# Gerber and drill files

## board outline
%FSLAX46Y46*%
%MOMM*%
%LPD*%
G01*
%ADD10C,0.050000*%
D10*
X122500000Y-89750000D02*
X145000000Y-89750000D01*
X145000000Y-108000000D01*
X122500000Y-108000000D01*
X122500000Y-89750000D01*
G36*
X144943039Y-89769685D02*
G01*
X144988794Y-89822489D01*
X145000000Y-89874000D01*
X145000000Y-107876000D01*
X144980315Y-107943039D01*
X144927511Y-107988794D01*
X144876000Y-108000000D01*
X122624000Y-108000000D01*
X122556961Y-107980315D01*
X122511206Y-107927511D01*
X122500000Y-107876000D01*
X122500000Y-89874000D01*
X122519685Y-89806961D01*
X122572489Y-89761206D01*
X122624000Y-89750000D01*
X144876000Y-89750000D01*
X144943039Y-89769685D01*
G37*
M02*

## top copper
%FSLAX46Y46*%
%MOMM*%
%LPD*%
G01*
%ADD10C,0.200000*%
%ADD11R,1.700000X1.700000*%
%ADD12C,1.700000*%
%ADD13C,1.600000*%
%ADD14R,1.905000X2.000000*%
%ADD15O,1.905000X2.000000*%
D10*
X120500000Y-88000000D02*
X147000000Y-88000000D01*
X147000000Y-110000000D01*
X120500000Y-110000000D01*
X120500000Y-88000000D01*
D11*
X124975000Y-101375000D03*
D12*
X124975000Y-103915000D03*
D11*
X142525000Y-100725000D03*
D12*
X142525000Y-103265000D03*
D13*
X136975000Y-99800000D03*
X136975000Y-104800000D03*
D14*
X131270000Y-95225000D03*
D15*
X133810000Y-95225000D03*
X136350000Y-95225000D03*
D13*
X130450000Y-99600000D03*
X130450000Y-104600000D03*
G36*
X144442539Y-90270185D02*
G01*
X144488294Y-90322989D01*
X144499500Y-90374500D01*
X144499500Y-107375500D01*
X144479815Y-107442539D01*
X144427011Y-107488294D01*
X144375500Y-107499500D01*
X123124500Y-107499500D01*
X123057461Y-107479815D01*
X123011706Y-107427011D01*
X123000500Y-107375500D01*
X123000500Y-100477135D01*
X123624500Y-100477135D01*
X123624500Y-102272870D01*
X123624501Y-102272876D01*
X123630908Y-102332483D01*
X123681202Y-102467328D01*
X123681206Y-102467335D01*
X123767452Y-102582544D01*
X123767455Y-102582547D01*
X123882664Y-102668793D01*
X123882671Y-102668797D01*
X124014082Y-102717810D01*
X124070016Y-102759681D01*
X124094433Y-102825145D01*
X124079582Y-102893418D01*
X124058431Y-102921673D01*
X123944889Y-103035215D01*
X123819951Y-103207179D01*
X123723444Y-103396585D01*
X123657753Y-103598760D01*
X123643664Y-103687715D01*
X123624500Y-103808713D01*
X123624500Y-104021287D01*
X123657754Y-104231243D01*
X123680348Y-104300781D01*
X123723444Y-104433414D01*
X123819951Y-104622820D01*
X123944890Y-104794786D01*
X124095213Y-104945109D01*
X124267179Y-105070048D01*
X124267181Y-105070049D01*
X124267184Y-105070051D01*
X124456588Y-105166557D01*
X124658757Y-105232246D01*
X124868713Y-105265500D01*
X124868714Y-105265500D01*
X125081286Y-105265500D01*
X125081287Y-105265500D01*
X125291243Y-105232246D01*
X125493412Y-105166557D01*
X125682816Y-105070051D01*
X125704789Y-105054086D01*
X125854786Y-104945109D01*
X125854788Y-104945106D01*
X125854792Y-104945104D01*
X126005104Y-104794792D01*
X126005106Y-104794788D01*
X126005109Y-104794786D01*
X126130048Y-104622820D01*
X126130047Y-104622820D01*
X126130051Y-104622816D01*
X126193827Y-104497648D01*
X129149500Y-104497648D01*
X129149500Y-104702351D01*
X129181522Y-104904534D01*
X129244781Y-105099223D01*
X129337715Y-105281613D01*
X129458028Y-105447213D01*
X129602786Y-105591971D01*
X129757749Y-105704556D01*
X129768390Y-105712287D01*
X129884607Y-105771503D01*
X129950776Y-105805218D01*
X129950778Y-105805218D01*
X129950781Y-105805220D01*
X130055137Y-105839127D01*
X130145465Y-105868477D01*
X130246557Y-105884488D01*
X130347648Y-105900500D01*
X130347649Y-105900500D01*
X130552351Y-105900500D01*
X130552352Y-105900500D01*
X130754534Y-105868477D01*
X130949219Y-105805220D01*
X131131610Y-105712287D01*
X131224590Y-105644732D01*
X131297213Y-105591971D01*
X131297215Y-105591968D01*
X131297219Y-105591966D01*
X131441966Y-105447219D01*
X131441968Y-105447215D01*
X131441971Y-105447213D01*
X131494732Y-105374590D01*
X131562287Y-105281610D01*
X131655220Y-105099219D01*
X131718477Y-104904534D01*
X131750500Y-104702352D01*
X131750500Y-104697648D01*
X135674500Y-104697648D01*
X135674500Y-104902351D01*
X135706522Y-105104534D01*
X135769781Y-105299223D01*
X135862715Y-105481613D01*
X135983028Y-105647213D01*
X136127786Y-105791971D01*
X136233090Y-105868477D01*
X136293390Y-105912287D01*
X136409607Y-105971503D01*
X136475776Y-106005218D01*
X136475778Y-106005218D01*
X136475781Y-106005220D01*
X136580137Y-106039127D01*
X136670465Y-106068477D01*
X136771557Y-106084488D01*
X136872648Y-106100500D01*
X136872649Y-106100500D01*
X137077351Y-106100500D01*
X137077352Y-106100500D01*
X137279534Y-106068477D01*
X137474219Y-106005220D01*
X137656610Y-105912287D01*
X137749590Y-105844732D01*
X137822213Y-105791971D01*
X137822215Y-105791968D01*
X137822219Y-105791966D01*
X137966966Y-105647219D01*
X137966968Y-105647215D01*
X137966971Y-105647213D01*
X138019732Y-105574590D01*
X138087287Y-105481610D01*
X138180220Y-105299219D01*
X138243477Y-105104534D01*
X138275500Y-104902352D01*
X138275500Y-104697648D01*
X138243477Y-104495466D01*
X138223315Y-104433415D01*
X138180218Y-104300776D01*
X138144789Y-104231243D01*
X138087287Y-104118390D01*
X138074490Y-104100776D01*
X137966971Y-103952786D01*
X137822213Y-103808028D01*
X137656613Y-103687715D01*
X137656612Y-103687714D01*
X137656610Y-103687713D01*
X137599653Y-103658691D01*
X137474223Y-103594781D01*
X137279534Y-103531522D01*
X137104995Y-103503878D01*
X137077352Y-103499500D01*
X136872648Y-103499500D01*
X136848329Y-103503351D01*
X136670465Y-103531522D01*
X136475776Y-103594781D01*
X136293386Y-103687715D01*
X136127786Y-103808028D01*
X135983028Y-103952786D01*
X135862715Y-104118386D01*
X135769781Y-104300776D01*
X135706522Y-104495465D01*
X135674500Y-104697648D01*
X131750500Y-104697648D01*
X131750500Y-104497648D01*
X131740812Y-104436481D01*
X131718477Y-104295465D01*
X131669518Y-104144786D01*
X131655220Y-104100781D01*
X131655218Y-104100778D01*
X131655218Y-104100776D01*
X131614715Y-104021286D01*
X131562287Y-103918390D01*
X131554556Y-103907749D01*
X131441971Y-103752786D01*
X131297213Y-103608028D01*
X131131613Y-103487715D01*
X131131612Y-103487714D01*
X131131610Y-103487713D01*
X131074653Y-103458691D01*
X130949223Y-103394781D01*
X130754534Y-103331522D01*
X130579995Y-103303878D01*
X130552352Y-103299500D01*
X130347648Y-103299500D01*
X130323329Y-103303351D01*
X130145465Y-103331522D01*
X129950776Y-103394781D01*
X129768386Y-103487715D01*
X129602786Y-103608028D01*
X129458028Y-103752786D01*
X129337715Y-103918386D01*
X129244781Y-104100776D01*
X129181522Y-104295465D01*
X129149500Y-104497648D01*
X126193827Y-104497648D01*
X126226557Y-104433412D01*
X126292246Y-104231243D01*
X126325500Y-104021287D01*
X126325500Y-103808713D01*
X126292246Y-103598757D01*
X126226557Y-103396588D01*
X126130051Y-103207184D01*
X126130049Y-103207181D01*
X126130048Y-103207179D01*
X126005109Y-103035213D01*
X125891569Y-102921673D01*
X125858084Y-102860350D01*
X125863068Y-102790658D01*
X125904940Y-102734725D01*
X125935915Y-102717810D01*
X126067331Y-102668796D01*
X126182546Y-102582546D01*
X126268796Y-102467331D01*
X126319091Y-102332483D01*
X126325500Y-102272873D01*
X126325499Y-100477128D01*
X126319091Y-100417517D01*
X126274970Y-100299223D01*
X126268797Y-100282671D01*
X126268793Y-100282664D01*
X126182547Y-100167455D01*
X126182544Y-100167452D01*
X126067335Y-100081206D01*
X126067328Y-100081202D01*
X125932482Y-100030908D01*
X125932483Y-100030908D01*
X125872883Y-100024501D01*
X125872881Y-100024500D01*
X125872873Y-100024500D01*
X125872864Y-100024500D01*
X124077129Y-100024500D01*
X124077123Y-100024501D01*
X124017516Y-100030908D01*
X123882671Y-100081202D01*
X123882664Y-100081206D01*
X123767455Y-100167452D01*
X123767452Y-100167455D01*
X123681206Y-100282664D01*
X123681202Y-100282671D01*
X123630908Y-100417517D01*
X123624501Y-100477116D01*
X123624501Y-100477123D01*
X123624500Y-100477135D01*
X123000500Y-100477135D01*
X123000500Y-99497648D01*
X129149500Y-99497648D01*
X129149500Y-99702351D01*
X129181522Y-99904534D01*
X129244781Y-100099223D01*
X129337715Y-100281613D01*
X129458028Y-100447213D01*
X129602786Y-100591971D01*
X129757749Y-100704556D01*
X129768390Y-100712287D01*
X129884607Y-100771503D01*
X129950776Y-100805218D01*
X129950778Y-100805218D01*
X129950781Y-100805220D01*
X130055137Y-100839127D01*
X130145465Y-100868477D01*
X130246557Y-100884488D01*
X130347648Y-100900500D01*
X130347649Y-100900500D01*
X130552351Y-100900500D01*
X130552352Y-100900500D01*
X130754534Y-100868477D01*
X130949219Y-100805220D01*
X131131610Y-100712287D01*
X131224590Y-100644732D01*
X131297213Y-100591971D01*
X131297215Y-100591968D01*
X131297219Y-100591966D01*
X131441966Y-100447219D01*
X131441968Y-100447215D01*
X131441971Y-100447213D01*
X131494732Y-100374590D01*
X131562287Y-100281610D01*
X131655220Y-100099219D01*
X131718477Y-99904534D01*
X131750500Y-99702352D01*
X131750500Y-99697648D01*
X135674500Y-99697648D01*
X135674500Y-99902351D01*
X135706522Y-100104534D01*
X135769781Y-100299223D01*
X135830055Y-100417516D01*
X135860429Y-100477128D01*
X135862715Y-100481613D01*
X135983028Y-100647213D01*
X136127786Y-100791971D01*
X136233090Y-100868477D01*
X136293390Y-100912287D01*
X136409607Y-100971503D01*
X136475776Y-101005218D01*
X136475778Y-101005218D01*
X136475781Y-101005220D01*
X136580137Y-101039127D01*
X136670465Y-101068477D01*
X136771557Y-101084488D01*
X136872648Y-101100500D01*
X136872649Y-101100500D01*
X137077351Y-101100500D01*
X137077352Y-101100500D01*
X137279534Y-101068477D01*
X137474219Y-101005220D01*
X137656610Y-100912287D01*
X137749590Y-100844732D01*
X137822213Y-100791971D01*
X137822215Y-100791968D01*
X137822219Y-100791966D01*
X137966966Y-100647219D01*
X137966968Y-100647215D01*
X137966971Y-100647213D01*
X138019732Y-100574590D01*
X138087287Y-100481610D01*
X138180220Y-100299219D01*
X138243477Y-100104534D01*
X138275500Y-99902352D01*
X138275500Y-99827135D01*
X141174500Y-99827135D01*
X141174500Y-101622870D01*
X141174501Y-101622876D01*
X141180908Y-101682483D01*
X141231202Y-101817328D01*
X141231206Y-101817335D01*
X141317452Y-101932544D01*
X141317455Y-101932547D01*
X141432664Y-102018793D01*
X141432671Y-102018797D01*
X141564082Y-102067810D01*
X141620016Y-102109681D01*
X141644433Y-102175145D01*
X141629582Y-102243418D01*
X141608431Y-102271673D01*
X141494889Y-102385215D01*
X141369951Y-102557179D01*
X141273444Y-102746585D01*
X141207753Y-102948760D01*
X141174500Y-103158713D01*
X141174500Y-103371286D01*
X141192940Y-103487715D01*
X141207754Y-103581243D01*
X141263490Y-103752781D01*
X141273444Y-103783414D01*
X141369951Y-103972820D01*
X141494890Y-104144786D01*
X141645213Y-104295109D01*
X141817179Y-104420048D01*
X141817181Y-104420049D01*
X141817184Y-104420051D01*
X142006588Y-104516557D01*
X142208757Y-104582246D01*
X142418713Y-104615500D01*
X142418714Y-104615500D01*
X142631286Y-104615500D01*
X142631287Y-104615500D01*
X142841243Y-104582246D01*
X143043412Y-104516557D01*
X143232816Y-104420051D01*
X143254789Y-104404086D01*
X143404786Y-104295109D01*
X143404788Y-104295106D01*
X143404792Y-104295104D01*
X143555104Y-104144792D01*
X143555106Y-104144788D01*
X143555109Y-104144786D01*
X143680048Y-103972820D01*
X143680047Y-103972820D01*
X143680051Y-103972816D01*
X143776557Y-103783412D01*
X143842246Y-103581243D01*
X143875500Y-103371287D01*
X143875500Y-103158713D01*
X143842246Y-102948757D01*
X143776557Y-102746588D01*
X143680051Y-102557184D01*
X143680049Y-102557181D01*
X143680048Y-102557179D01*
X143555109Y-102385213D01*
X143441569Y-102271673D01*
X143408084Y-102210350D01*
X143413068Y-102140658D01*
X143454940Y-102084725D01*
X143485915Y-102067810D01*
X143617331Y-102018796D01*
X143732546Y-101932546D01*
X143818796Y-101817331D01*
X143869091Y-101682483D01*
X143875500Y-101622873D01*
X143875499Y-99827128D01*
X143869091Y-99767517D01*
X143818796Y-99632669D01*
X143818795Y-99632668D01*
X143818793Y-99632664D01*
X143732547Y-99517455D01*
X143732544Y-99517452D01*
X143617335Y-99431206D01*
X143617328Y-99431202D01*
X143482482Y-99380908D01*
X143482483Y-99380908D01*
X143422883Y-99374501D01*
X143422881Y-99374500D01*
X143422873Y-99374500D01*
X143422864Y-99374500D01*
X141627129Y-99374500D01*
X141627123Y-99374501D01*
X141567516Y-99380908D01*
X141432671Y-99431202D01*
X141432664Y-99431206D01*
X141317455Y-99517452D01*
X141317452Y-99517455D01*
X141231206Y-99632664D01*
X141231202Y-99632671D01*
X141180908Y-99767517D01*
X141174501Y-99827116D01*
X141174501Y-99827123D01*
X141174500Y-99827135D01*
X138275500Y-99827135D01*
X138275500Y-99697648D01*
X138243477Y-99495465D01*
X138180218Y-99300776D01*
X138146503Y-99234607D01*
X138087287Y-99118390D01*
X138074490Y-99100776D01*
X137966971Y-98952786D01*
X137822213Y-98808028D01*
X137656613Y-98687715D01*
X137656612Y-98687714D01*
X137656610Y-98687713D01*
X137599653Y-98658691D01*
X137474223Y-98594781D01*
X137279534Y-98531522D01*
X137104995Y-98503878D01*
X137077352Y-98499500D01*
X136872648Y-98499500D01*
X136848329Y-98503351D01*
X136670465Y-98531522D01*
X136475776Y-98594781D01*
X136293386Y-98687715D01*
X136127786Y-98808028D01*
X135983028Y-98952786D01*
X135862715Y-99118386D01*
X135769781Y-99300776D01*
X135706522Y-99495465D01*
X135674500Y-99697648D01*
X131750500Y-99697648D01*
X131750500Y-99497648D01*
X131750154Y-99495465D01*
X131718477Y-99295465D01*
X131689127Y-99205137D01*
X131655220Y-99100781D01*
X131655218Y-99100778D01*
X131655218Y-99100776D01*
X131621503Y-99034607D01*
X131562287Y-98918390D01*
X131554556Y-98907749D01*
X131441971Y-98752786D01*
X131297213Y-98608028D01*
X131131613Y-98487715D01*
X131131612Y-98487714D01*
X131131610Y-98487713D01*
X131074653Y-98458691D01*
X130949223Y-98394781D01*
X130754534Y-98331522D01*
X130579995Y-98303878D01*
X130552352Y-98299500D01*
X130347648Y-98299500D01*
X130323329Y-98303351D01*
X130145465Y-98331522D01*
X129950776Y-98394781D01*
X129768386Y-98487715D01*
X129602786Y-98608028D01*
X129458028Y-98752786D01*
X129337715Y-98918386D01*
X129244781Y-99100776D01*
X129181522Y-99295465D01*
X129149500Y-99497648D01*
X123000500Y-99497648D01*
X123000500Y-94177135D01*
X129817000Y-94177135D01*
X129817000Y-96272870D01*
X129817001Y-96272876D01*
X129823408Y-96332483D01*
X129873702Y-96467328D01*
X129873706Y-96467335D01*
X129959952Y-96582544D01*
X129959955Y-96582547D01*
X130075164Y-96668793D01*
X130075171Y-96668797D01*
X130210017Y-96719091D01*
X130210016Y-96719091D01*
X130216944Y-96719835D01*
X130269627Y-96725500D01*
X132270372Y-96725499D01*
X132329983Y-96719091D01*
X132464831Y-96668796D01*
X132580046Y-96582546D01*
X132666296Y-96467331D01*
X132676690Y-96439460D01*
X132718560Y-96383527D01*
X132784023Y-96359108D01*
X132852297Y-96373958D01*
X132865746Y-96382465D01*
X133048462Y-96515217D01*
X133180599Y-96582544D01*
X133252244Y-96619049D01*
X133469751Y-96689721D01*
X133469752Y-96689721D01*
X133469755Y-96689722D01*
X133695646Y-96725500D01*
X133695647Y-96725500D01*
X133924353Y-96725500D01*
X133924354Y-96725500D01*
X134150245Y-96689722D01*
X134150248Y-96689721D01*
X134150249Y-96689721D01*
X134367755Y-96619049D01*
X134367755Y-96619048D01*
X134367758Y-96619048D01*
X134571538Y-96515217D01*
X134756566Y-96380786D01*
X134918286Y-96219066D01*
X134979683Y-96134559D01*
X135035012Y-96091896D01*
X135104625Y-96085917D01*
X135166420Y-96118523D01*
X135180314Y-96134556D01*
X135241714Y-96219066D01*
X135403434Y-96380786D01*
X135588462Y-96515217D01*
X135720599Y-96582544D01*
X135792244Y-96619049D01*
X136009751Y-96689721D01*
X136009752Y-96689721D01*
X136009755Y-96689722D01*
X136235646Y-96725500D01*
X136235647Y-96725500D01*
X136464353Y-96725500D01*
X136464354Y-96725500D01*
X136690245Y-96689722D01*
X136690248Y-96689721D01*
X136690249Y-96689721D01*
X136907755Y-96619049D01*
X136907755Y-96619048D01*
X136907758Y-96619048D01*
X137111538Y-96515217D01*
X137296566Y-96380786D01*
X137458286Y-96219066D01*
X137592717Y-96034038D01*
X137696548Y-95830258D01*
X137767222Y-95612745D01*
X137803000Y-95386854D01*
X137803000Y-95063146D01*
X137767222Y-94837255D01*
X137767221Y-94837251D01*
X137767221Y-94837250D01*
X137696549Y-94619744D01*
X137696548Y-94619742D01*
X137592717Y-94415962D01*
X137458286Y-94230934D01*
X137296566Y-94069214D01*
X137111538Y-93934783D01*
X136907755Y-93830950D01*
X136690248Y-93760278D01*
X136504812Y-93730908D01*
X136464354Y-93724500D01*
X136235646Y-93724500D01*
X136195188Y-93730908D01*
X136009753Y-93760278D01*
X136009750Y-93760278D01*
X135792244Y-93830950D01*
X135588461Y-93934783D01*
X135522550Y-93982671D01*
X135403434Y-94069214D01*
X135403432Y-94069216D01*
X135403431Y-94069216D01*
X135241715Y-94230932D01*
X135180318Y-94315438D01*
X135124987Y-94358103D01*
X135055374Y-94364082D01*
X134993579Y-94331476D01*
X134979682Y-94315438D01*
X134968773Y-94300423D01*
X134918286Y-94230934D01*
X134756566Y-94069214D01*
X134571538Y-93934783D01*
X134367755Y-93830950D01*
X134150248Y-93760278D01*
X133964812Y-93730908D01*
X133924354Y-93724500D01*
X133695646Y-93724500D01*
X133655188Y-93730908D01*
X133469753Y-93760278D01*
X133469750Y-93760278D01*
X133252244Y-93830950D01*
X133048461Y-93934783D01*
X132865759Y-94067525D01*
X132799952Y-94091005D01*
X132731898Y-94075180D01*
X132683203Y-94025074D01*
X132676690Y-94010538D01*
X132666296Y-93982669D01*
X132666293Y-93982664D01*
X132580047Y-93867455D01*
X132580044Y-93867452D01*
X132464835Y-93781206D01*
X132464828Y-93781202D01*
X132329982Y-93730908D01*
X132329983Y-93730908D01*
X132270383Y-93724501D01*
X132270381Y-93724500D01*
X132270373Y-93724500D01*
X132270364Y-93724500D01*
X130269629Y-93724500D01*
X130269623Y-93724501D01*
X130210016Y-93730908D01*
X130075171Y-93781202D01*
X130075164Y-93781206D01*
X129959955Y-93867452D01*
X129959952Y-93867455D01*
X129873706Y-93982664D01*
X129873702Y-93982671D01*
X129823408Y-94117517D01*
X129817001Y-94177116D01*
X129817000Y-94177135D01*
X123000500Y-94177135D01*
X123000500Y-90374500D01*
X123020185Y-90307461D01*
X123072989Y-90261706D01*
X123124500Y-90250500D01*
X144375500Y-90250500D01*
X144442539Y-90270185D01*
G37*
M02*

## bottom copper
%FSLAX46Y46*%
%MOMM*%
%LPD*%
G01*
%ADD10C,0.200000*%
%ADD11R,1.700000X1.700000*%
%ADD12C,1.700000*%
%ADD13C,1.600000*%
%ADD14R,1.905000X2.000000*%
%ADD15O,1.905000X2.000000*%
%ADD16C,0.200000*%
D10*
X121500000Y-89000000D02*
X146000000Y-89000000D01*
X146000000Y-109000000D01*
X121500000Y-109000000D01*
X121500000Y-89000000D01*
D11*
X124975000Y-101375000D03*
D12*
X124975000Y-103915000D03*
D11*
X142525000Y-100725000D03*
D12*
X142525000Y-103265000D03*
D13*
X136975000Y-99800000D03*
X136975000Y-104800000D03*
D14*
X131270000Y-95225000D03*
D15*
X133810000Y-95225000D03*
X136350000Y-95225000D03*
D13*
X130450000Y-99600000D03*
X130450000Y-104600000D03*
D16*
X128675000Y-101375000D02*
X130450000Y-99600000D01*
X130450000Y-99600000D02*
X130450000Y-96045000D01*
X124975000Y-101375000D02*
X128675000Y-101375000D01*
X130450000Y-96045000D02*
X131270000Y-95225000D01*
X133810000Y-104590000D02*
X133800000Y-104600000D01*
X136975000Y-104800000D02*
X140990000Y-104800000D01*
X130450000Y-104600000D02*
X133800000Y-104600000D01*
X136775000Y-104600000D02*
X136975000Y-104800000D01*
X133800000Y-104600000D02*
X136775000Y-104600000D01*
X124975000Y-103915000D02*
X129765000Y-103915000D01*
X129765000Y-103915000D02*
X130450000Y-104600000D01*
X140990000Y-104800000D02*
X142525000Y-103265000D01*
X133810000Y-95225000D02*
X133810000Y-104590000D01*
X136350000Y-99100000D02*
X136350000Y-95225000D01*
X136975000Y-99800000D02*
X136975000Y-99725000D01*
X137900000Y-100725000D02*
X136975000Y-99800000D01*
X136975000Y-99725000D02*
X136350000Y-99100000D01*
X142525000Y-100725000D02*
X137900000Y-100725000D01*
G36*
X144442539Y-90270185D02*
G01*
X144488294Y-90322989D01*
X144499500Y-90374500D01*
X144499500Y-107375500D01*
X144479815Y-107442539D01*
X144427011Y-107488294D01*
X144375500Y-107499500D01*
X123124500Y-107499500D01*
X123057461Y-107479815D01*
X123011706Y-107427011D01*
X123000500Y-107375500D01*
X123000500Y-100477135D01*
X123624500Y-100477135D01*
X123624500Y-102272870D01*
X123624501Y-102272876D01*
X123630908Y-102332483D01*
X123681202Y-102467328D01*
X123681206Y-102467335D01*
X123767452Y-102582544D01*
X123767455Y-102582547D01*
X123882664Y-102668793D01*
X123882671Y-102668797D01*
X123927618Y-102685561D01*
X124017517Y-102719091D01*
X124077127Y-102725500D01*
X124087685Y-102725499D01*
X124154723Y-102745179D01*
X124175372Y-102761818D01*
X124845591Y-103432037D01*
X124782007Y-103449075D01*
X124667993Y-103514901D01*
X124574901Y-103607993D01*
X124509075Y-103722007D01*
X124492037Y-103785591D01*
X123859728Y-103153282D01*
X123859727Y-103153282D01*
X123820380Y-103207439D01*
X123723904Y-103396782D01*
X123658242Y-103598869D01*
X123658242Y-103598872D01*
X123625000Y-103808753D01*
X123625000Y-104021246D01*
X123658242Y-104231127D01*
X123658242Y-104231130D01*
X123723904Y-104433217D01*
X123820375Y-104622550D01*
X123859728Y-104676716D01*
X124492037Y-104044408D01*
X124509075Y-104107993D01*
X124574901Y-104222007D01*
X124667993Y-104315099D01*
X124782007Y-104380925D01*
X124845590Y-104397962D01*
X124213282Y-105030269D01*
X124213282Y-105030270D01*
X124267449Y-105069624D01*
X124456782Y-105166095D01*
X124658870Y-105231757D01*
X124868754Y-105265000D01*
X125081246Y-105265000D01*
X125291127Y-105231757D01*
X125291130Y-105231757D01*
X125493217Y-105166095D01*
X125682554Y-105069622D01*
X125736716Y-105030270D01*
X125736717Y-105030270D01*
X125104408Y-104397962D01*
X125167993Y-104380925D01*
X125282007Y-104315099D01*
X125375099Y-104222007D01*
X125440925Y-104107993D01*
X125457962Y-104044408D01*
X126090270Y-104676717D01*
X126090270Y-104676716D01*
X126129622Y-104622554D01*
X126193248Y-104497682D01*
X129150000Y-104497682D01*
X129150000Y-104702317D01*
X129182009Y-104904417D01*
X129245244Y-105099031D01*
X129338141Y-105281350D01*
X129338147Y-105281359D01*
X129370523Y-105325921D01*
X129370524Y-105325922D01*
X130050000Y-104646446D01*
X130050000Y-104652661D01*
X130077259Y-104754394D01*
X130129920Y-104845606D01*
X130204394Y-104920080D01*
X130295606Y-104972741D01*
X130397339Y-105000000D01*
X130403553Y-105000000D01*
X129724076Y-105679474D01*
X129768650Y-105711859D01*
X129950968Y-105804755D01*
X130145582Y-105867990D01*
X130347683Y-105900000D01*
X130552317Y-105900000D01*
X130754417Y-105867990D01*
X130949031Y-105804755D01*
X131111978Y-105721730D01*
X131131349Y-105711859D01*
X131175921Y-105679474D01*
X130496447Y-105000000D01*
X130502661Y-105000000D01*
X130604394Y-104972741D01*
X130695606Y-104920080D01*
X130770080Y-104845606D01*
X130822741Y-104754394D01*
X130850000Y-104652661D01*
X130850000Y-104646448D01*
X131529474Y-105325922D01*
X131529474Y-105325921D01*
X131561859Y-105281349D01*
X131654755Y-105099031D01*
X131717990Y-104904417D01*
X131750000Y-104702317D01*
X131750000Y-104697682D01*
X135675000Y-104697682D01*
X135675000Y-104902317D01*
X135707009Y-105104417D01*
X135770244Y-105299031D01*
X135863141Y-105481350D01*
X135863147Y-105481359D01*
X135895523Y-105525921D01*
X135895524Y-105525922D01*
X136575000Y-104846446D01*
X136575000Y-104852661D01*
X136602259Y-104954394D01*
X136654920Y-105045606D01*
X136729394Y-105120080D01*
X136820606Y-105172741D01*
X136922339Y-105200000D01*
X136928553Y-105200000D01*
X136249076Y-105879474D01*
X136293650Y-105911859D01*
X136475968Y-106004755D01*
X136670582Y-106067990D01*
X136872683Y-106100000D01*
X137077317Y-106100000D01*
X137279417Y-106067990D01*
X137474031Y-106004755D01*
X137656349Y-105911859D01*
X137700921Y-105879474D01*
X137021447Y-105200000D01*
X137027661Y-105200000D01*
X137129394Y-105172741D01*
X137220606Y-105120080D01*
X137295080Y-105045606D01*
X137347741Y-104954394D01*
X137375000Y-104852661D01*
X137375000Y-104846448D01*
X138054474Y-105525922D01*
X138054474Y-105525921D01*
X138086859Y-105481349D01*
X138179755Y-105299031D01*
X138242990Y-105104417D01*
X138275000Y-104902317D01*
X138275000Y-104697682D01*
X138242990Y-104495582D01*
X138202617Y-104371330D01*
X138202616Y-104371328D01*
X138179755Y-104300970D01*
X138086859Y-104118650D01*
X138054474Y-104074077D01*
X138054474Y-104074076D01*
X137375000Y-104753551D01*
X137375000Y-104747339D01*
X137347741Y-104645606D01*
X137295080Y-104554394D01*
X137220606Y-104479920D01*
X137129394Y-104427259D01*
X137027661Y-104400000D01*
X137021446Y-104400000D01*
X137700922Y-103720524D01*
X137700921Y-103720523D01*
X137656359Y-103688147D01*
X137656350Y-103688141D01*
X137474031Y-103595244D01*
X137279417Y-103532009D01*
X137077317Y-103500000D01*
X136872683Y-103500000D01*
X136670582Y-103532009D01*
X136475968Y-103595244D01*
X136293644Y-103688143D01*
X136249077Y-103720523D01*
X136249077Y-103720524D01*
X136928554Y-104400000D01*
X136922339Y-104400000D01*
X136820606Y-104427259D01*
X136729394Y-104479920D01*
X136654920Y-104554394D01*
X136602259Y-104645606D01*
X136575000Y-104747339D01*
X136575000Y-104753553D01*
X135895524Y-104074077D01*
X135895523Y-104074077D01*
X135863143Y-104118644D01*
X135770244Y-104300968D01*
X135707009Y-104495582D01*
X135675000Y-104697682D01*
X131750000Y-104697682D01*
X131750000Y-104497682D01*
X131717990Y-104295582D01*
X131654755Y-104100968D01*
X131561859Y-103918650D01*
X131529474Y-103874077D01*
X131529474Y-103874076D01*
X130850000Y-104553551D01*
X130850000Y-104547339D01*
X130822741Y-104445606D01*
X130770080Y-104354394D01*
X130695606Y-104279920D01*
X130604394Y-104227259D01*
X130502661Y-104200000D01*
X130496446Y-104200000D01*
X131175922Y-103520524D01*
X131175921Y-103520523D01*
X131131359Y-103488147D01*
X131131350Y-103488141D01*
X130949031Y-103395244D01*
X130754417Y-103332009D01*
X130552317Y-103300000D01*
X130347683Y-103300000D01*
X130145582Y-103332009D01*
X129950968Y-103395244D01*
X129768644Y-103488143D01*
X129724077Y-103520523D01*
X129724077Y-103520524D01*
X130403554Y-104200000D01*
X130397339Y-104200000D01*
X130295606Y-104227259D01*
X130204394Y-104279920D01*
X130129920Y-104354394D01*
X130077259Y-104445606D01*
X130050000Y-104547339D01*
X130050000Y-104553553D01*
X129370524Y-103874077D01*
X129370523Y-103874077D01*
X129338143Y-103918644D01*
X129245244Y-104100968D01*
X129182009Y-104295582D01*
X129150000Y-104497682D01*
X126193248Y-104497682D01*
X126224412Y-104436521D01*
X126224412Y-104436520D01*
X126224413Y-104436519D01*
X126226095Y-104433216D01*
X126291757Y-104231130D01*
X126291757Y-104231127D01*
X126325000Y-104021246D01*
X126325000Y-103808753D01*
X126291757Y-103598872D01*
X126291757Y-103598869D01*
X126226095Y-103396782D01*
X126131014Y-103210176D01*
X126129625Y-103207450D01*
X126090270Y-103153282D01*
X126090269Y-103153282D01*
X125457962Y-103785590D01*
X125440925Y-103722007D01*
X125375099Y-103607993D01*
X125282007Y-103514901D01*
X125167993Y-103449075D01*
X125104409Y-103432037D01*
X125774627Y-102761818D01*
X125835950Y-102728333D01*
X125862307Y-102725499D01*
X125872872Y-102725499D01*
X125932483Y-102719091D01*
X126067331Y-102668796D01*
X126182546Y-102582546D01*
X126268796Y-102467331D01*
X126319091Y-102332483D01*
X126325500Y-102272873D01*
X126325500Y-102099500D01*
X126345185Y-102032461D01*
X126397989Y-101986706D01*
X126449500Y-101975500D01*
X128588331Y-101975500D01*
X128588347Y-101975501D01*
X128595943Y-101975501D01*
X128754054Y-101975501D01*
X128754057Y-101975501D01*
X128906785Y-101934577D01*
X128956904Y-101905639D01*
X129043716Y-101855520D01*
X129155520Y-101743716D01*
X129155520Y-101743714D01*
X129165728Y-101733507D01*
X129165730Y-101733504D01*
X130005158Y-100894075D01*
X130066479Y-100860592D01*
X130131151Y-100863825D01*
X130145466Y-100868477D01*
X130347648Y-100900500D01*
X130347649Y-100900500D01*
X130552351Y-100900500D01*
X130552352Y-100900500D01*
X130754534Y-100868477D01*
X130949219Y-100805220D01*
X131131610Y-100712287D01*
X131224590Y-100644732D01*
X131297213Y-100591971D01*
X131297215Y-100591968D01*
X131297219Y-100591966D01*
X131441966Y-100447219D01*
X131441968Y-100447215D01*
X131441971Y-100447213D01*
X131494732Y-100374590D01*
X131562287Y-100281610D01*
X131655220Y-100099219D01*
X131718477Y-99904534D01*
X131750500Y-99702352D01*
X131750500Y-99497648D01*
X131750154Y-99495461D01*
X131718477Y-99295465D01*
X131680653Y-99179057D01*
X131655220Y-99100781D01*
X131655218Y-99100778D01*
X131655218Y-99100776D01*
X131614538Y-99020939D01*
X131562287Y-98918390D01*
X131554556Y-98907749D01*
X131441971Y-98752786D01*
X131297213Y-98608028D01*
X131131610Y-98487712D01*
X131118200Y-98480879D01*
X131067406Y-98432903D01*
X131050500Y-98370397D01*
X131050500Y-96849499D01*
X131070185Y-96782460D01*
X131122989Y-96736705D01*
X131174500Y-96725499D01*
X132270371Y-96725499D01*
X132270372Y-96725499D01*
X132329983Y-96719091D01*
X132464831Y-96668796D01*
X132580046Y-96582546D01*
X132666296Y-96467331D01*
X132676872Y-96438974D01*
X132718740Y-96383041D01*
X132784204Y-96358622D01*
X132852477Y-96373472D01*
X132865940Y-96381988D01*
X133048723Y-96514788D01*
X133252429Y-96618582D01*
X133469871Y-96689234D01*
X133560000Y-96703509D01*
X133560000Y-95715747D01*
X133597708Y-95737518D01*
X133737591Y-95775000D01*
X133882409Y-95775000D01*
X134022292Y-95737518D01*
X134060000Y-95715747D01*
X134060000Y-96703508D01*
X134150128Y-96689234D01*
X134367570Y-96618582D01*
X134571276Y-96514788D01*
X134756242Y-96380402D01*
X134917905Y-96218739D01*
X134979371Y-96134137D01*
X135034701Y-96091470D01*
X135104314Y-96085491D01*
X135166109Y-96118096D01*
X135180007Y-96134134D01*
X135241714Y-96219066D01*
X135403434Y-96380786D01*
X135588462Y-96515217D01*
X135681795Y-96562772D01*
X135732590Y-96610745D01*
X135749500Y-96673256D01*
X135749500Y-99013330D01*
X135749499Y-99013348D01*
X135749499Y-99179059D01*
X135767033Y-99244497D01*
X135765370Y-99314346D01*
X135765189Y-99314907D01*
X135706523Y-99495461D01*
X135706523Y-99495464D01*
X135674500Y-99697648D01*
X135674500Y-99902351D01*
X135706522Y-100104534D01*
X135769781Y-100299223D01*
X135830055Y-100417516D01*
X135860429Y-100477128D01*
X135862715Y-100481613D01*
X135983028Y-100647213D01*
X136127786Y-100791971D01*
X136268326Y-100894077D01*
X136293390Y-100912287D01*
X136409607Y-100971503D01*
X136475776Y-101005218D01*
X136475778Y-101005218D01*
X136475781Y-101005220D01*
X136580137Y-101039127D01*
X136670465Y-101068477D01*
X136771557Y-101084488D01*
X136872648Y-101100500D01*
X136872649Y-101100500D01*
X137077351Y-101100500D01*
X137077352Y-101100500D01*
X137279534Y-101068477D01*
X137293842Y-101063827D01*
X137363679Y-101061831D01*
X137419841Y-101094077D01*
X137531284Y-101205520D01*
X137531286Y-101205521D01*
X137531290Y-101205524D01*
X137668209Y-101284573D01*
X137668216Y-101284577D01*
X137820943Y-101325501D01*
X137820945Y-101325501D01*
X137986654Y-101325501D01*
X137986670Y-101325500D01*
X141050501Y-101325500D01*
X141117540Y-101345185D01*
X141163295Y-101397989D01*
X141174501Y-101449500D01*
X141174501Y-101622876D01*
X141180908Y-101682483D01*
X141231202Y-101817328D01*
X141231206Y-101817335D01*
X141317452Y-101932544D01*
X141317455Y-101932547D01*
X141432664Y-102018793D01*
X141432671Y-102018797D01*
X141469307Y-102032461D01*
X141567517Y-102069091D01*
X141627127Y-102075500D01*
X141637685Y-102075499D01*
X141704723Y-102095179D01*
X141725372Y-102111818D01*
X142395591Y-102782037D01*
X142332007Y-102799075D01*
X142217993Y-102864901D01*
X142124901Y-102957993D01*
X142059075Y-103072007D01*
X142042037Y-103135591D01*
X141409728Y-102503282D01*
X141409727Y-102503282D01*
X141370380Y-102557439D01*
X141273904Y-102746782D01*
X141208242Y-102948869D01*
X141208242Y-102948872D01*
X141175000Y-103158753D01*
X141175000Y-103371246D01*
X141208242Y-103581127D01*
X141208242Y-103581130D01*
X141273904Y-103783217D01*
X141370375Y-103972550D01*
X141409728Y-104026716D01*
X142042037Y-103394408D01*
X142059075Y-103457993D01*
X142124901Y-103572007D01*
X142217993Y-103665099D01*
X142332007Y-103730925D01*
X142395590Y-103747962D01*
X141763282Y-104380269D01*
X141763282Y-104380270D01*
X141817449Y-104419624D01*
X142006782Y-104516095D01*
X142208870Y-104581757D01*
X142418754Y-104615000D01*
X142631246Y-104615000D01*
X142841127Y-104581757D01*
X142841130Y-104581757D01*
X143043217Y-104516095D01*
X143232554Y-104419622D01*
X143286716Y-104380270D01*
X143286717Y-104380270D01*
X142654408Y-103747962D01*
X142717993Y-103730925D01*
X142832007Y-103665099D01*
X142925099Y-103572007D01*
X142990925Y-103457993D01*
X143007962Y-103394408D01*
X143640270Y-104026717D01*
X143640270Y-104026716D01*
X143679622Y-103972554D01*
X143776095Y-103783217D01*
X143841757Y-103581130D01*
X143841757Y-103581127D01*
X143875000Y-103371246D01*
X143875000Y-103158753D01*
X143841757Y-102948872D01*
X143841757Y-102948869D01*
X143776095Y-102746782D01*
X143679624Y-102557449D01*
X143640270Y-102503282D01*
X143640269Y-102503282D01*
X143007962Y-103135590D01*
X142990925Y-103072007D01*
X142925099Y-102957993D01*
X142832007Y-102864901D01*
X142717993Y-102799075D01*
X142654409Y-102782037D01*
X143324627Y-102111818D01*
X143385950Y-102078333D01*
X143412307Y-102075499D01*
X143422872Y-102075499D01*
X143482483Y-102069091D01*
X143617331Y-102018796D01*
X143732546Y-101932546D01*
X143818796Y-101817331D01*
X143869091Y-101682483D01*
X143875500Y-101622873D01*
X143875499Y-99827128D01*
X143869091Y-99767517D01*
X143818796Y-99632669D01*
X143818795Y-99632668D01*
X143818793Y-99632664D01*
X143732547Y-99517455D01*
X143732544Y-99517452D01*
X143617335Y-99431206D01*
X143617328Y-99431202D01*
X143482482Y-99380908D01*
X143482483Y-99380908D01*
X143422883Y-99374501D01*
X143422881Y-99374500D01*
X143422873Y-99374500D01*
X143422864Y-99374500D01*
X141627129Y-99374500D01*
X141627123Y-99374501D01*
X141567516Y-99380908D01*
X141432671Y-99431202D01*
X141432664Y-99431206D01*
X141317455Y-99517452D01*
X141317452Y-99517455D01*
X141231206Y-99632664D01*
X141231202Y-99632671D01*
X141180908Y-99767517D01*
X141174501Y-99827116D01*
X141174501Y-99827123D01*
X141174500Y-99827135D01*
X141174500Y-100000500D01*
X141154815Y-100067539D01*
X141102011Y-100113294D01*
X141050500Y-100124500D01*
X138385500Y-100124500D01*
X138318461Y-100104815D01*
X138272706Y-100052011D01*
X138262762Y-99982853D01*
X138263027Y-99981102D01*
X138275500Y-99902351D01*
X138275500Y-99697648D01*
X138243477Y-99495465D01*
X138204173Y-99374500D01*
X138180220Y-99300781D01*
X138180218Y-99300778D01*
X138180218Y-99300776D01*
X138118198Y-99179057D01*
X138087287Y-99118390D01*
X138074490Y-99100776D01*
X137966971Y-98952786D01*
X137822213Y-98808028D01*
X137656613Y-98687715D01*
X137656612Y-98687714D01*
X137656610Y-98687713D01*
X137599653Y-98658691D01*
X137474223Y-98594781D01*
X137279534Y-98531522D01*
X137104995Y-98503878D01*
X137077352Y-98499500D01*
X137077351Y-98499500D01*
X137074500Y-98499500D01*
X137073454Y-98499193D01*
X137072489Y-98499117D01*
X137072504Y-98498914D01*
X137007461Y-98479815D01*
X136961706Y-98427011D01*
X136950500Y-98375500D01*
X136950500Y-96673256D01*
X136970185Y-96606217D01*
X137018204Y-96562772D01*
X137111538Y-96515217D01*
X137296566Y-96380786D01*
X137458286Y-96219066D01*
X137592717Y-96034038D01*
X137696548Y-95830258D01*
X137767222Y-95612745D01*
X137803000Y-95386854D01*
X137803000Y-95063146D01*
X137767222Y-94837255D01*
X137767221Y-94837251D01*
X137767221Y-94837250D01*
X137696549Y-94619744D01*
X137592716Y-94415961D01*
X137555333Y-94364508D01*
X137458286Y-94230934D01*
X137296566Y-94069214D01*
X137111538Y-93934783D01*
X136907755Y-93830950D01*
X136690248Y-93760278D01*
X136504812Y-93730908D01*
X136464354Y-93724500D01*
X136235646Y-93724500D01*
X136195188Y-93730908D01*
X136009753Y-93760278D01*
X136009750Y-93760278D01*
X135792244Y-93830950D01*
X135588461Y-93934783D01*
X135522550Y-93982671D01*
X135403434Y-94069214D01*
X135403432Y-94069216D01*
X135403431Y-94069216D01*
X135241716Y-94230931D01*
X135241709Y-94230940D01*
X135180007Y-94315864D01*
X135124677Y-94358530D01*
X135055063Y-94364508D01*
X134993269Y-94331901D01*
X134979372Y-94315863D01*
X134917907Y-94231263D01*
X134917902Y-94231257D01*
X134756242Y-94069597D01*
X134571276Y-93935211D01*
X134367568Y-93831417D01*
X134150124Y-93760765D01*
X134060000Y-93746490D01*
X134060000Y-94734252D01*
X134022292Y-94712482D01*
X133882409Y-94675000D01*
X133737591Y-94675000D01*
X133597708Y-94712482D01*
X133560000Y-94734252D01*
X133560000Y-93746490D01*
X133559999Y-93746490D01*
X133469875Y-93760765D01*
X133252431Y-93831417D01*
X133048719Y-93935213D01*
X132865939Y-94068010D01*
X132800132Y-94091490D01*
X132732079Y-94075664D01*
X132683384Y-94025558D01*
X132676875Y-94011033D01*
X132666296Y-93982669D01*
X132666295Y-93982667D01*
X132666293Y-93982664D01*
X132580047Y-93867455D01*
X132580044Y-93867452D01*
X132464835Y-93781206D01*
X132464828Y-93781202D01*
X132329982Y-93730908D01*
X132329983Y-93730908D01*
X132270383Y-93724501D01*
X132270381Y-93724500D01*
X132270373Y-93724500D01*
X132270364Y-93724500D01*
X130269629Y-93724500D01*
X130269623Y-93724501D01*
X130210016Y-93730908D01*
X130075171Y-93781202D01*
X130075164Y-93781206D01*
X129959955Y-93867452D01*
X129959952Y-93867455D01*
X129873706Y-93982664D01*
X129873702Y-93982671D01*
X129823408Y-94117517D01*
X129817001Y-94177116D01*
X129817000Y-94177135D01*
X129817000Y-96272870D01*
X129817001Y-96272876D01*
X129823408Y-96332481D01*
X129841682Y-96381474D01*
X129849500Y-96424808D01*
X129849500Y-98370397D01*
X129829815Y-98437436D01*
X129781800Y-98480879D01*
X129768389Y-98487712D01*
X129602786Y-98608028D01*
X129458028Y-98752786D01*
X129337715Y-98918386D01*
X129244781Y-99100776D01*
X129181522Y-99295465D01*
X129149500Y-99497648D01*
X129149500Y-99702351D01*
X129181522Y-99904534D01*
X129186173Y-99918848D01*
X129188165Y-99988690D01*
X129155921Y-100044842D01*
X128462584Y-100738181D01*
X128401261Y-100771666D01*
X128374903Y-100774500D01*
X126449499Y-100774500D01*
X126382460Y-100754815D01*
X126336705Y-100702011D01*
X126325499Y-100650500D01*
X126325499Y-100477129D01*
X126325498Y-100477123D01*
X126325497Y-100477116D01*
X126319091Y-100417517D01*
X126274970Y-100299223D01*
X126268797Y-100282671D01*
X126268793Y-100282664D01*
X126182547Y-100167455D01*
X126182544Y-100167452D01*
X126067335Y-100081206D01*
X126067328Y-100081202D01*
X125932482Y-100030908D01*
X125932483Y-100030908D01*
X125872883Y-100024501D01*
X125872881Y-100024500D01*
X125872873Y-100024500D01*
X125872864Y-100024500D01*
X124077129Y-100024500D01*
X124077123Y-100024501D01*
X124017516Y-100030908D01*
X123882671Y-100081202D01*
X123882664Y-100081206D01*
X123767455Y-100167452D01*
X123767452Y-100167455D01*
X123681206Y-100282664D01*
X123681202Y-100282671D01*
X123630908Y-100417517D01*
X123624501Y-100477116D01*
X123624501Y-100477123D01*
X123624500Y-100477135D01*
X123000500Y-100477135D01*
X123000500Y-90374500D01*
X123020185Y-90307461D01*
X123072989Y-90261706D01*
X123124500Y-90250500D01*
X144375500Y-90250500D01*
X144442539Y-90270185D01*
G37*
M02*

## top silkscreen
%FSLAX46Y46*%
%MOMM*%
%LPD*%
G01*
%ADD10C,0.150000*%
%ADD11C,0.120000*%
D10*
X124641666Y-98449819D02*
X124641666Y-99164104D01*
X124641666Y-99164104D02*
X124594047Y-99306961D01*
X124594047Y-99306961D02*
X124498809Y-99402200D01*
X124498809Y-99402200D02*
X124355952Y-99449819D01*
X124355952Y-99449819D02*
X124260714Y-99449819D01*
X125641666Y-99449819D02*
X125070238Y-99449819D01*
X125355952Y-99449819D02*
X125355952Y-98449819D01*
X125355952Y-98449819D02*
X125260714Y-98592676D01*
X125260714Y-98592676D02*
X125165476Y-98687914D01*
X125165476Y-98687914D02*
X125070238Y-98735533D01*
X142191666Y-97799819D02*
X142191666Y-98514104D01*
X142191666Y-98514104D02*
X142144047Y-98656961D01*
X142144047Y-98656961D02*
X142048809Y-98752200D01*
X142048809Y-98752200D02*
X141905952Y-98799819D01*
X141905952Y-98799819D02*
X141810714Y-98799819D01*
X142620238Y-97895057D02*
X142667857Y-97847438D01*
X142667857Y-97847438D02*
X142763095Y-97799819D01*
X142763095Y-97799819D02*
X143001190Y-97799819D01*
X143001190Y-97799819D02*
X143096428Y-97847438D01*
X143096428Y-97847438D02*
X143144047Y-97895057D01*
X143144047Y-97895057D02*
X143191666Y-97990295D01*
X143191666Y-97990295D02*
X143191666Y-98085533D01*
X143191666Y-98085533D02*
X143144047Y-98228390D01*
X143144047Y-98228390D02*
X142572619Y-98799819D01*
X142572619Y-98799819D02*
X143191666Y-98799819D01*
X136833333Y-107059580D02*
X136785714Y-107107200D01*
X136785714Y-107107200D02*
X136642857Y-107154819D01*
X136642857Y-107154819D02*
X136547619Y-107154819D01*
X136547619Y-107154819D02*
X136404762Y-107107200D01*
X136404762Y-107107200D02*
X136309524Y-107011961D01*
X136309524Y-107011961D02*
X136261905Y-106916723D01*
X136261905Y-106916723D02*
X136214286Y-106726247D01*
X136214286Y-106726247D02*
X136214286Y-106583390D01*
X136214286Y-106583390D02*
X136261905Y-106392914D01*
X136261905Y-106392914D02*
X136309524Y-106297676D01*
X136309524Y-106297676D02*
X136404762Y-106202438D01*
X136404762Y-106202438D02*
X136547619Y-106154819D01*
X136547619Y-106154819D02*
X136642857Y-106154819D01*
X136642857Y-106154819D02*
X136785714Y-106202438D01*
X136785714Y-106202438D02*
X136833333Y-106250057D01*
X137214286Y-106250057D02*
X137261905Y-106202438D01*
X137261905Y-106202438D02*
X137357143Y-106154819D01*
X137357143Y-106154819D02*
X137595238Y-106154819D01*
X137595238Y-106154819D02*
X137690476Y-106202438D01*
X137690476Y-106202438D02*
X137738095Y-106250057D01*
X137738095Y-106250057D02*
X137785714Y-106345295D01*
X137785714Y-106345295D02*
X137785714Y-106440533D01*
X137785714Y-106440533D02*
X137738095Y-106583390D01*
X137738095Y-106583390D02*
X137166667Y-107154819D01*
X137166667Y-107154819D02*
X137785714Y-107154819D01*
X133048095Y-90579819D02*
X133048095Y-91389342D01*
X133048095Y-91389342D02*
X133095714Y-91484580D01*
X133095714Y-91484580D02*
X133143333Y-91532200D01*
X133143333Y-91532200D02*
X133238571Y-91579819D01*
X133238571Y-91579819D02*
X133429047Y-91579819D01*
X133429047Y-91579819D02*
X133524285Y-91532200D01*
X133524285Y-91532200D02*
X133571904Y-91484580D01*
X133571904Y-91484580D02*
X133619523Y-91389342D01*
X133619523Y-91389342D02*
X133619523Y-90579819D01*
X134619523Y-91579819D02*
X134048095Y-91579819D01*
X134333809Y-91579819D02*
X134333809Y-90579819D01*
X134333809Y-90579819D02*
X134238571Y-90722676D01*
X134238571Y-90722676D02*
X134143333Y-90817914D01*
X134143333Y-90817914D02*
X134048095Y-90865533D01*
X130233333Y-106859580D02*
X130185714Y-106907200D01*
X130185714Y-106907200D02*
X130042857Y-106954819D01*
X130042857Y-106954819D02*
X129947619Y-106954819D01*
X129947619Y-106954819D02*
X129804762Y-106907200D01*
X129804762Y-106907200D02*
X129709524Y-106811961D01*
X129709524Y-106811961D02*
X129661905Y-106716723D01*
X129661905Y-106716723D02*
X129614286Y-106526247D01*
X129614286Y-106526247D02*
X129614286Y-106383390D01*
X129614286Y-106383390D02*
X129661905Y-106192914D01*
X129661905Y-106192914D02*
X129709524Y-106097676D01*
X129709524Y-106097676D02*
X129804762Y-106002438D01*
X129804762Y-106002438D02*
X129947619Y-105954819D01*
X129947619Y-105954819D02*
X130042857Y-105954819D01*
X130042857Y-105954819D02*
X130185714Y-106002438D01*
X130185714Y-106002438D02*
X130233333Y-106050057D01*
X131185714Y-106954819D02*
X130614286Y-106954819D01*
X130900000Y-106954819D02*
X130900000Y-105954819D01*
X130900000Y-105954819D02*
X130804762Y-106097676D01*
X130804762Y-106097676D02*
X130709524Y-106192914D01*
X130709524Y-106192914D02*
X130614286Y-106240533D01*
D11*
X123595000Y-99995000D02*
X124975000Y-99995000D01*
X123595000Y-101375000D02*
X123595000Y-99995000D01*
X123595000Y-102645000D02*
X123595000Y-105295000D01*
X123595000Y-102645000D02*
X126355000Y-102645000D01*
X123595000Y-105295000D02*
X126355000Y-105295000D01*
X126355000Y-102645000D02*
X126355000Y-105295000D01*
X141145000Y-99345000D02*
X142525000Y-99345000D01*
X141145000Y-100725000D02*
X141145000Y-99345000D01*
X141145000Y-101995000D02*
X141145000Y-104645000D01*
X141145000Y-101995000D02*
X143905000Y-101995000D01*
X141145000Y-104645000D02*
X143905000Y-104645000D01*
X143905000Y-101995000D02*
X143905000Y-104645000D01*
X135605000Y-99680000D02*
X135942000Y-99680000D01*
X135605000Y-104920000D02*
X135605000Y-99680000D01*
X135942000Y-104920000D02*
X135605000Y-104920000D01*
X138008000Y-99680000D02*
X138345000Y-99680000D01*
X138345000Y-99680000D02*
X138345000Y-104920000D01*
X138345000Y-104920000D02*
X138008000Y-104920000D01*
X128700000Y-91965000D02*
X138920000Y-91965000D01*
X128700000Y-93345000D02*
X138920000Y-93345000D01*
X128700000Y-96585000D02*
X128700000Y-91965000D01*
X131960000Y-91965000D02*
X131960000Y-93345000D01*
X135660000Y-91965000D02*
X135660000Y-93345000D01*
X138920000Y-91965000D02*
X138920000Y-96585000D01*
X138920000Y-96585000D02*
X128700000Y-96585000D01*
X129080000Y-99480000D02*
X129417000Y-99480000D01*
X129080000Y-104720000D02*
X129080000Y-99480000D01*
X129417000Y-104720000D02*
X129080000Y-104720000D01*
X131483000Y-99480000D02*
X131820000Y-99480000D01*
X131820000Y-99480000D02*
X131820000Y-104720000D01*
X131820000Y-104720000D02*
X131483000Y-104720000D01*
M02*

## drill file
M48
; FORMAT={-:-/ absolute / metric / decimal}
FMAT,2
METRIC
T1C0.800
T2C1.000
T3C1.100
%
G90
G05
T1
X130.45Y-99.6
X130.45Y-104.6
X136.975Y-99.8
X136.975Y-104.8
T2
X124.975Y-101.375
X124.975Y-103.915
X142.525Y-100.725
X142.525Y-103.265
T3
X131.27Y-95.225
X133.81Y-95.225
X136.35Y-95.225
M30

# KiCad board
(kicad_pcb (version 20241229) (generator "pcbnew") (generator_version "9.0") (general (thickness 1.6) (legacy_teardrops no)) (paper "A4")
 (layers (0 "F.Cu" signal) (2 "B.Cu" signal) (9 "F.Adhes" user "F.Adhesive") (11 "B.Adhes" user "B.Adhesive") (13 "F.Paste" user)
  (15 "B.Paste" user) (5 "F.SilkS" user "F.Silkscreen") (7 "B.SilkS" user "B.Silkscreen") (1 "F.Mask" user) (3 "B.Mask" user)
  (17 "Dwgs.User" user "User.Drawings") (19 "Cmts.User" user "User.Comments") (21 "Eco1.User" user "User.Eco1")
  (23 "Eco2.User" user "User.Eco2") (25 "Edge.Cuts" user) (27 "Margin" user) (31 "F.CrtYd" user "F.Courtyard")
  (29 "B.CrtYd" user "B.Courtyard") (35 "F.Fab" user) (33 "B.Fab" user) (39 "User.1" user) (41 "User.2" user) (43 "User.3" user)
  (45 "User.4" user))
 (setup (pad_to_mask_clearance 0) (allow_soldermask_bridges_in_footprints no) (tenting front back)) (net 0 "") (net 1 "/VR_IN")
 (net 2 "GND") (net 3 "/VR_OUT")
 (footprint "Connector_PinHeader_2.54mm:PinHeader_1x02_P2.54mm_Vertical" (layer "F.Cu") (at 124.975 101.375)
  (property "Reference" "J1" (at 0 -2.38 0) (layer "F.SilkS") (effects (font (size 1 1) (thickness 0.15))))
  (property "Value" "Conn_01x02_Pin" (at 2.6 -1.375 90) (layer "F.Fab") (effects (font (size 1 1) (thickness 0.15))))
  (fp_line (start -1.38 -1.38) (end 0 -1.38) (stroke (width 0.12) (type solid)) (layer "F.SilkS"))
  (fp_line (start -1.38 0) (end -1.38 -1.38) (stroke (width 0.12) (type solid)) (layer "F.SilkS"))
  (fp_line (start -1.38 1.27) (end -1.38 3.92) (stroke (width 0.12) (type solid)) (layer "F.SilkS"))
  (fp_line (start -1.38 1.27) (end 1.38 1.27) (stroke (width 0.12) (type solid)) (layer "F.SilkS"))
  (fp_line (start -1.38 3.92) (end 1.38 3.92) (stroke (width 0.12) (type solid)) (layer "F.SilkS"))
  (fp_line (start 1.38 1.27) (end 1.38 3.92) (stroke (width 0.12) (type solid)) (layer "F.SilkS"))
  (pad "1" thru_hole rect (at 0 0) (size 1.7 1.7) (drill 1) (layers "*.Cu" "*.Mask") (remove_unused_layers no) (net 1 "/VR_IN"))
  (pad "2" thru_hole circle (at 0 2.54) (size 1.7 1.7) (drill 1) (layers "*.Cu" "*.Mask") (remove_unused_layers no) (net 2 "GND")))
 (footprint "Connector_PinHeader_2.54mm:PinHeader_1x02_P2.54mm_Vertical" (layer "F.Cu") (at 142.525 100.725)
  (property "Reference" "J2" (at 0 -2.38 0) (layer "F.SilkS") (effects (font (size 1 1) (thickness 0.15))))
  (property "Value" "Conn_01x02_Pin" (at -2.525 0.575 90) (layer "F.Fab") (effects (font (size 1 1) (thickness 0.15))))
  (fp_line (start -1.38 -1.38) (end 0 -1.38) (stroke (width 0.12) (type solid)) (layer "F.SilkS"))
  (fp_line (start -1.38 0) (end -1.38 -1.38) (stroke (width 0.12) (type solid)) (layer "F.SilkS"))
  (fp_line (start -1.38 1.27) (end -1.38 3.92) (stroke (width 0.12) (type solid)) (layer "F.SilkS"))
  (fp_line (start -1.38 1.27) (end 1.38 1.27) (stroke (width 0.12) (type solid)) (layer "F.SilkS"))
  (fp_line (start -1.38 3.92) (end 1.38 3.92) (stroke (width 0.12) (type solid)) (layer "F.SilkS"))
  (fp_line (start 1.38 1.27) (end 1.38 3.92) (stroke (width 0.12) (type solid)) (layer "F.SilkS"))
  (pad "1" thru_hole rect (at 0 0) (size 1.7 1.7) (drill 1) (layers "*.Cu" "*.Mask") (remove_unused_layers no) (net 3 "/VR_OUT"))
  (pad "2" thru_hole circle (at 0 2.54) (size 1.7 1.7) (drill 1) (layers "*.Cu" "*.Mask") (remove_unused_layers no) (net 2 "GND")))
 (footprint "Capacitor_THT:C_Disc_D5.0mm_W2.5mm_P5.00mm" (layer "F.Cu") (at 136.975 99.8 -90)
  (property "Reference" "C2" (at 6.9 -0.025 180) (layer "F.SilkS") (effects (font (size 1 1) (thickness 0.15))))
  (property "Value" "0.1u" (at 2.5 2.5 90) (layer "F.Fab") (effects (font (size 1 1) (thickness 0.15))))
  (fp_line (start -0.12 1.37) (end -0.12 1.033) (stroke (width 0.12) (type solid)) (layer "F.SilkS"))
  (fp_line (start 5.12 1.37) (end -0.12 1.37) (stroke (width 0.12) (type solid)) (layer "F.SilkS"))
  (fp_line (start 5.12 1.033) (end 5.12 1.37) (stroke (width 0.12) (type solid)) (layer "F.SilkS"))
  (fp_line (start -0.12 -1.033) (end -0.12 -1.37) (stroke (width 0.12) (type solid)) (layer "F.SilkS"))
  (fp_line (start -0.12 -1.37) (end 5.12 -1.37) (stroke (width 0.12) (type solid)) (layer "F.SilkS"))
  (fp_line (start 5.12 -1.37) (end 5.12 -1.033) (stroke (width 0.12) (type solid)) (layer "F.SilkS"))
  (pad "1" thru_hole circle (at 0 0 270) (size 1.6 1.6) (drill 0.8) (layers "*.Cu" "*.Mask") (remove_unused_layers no) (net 3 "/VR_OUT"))
  (pad "2" thru_hole circle (at 5 0 270) (size 1.6 1.6) (drill 0.8) (layers "*.Cu" "*.Mask") (remove_unused_layers no) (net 2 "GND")))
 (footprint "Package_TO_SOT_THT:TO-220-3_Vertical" (layer "F.Cu") (at 131.27 95.225)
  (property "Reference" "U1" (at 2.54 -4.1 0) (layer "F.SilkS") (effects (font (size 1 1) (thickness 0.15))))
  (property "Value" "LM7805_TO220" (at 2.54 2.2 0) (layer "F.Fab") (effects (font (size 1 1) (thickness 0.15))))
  (fp_line (start -2.57 -3.26) (end 7.65 -3.26) (stroke (width 0.12) (type solid)) (layer "F.SilkS"))
  (fp_line (start -2.57 -1.88) (end 7.65 -1.88) (stroke (width 0.12) (type solid)) (layer "F.SilkS"))
  (fp_line (start -2.57 1.36) (end -2.57 -3.26) (stroke (width 0.12) (type solid)) (layer "F.SilkS"))
  (fp_line (start 0.69 -3.26) (end 0.69 -1.88) (stroke (width 0.12) (type solid)) (layer "F.SilkS"))
  (fp_line (start 4.39 -3.26) (end 4.39 -1.88) (stroke (width 0.12) (type solid)) (layer "F.SilkS"))
  (fp_line (start 7.65 -3.26) (end 7.65 1.36) (stroke (width 0.12) (type solid)) (layer "F.SilkS"))
  (fp_line (start 7.65 1.36) (end -2.57 1.36) (stroke (width 0.12) (type solid)) (layer "F.SilkS"))
  (pad "1" thru_hole rect (at 0 0) (size 1.905 2) (drill 1.1) (layers "*.Cu" "*.Mask") (remove_unused_layers no) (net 1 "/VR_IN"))
  (pad "2" thru_hole oval (at 2.54 0) (size 1.905 2) (drill 1.1) (layers "*.Cu" "*.Mask") (remove_unused_layers no) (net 2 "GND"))
  (pad "3" thru_hole oval (at 5.08 0) (size 1.905 2) (drill 1.1) (layers "*.Cu" "*.Mask") (remove_unused_layers no) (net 3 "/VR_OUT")))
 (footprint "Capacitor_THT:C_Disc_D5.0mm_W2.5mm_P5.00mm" (layer "F.Cu") (at 130.45 99.6 -90)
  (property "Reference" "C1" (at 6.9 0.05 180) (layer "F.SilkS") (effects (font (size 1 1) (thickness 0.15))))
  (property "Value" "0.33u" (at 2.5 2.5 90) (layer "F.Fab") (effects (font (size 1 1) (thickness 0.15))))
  (fp_line (start -0.12 1.37) (end -0.12 1.033) (stroke (width 0.12) (type solid)) (layer "F.SilkS"))
  (fp_line (start 5.12 1.37) (end -0.12 1.37) (stroke (width 0.12) (type solid)) (layer "F.SilkS"))
  (fp_line (start 5.12 1.033) (end 5.12 1.37) (stroke (width 0.12) (type solid)) (layer "F.SilkS"))
  (fp_line (start -0.12 -1.033) (end -0.12 -1.37) (stroke (width 0.12) (type solid)) (layer "F.SilkS"))
  (fp_line (start -0.12 -1.37) (end 5.12 -1.37) (stroke (width 0.12) (type solid)) (layer "F.SilkS"))
  (fp_line (start 5.12 -1.37) (end 5.12 -1.033) (stroke (width 0.12) (type solid)) (layer "F.SilkS"))
  (pad "1" thru_hole circle (at 0 0 270) (size 1.6 1.6) (drill 0.8) (layers "*.Cu" "*.Mask") (remove_unused_layers no) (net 1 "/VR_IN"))
  (pad "2" thru_hole circle (at 5 0 270) (size 1.6 1.6) (drill 0.8) (layers "*.Cu" "*.Mask") (remove_unused_layers no) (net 2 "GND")))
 (gr_rect (start 120.5 88) (end 147 110) (stroke (width 0.2) (type default)) (fill no) (layer "F.Cu"))
 (gr_rect (start 121.5 89) (end 146 109) (stroke (width 0.2) (type default)) (fill no) (layer "B.Cu"))
 (gr_rect (start 122.5 89.75) (end 145 108) (stroke (width 0.05) (type default)) (fill no) (layer "Edge.Cuts"))
 (segment (start 128.675 101.375) (end 130.45 99.6) (width 0.2) (layer "B.Cu") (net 1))
 (segment (start 130.45 99.6) (end 130.45 96.045) (width 0.2) (layer "B.Cu") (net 1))
 (segment (start 124.975 101.375) (end 128.675 101.375) (width 0.2) (layer "B.Cu") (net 1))
 (segment (start 130.45 96.045) (end 131.27 95.225) (width 0.2) (layer "B.Cu") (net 1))
 (segment (start 133.81 104.59) (end 133.8 104.6) (width 0.2) (layer "B.Cu") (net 2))
 (segment (start 136.975 104.8) (end 140.99 104.8) (width 0.2) (layer "B.Cu") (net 2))
 (segment (start 130.45 104.6) (end 133.8 104.6) (width 0.2) (layer "B.Cu") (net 2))
 (segment (start 136.775 104.6) (end 136.975 104.8) (width 0.2) (layer "B.Cu") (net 2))
 (segment (start 133.8 104.6) (end 136.775 104.6) (width 0.2) (layer "B.Cu") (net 2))
 (segment (start 124.975 103.915) (end 129.765 103.915) (width 0.2) (layer "B.Cu") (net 2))
 (segment (start 129.765 103.915) (end 130.45 104.6) (width 0.2) (layer "B.Cu") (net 2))
 (segment (start 140.99 104.8) (end 142.525 103.265) (width 0.2) (layer "B.Cu") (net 2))
 (segment (start 133.81 95.225) (end 133.81 104.59) (width 0.2) (layer "B.Cu") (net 2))
 (segment (start 136.35 99.1) (end 136.35 95.225) (width 0.2) (layer "B.Cu") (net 3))
 (segment (start 136.975 99.8) (end 136.975 99.725) (width 0.2) (layer "B.Cu") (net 3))
 (segment (start 137.9 100.725) (end 136.975 99.8) (width 0.2) (layer "B.Cu") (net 3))
 (segment (start 136.975 99.725) (end 136.35 99.1) (width 0.2) (layer "B.Cu") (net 3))
 (segment (start 142.525 100.725) (end 137.9 100.725) (width 0.2) (layer "B.Cu") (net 3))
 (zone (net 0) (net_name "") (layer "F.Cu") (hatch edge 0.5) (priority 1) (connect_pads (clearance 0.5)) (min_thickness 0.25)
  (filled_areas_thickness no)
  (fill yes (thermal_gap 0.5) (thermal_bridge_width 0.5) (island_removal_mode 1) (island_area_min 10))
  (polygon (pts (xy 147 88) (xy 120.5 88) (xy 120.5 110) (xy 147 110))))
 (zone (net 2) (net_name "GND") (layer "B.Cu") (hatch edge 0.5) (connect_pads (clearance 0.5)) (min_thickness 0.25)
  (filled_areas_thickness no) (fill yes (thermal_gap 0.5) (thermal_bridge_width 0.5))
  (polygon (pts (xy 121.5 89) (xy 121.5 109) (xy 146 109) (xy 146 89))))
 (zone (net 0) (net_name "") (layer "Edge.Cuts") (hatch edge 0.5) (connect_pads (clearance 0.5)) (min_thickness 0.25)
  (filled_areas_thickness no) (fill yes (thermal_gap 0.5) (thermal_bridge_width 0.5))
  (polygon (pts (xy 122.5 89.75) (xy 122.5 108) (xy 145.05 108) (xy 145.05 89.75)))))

